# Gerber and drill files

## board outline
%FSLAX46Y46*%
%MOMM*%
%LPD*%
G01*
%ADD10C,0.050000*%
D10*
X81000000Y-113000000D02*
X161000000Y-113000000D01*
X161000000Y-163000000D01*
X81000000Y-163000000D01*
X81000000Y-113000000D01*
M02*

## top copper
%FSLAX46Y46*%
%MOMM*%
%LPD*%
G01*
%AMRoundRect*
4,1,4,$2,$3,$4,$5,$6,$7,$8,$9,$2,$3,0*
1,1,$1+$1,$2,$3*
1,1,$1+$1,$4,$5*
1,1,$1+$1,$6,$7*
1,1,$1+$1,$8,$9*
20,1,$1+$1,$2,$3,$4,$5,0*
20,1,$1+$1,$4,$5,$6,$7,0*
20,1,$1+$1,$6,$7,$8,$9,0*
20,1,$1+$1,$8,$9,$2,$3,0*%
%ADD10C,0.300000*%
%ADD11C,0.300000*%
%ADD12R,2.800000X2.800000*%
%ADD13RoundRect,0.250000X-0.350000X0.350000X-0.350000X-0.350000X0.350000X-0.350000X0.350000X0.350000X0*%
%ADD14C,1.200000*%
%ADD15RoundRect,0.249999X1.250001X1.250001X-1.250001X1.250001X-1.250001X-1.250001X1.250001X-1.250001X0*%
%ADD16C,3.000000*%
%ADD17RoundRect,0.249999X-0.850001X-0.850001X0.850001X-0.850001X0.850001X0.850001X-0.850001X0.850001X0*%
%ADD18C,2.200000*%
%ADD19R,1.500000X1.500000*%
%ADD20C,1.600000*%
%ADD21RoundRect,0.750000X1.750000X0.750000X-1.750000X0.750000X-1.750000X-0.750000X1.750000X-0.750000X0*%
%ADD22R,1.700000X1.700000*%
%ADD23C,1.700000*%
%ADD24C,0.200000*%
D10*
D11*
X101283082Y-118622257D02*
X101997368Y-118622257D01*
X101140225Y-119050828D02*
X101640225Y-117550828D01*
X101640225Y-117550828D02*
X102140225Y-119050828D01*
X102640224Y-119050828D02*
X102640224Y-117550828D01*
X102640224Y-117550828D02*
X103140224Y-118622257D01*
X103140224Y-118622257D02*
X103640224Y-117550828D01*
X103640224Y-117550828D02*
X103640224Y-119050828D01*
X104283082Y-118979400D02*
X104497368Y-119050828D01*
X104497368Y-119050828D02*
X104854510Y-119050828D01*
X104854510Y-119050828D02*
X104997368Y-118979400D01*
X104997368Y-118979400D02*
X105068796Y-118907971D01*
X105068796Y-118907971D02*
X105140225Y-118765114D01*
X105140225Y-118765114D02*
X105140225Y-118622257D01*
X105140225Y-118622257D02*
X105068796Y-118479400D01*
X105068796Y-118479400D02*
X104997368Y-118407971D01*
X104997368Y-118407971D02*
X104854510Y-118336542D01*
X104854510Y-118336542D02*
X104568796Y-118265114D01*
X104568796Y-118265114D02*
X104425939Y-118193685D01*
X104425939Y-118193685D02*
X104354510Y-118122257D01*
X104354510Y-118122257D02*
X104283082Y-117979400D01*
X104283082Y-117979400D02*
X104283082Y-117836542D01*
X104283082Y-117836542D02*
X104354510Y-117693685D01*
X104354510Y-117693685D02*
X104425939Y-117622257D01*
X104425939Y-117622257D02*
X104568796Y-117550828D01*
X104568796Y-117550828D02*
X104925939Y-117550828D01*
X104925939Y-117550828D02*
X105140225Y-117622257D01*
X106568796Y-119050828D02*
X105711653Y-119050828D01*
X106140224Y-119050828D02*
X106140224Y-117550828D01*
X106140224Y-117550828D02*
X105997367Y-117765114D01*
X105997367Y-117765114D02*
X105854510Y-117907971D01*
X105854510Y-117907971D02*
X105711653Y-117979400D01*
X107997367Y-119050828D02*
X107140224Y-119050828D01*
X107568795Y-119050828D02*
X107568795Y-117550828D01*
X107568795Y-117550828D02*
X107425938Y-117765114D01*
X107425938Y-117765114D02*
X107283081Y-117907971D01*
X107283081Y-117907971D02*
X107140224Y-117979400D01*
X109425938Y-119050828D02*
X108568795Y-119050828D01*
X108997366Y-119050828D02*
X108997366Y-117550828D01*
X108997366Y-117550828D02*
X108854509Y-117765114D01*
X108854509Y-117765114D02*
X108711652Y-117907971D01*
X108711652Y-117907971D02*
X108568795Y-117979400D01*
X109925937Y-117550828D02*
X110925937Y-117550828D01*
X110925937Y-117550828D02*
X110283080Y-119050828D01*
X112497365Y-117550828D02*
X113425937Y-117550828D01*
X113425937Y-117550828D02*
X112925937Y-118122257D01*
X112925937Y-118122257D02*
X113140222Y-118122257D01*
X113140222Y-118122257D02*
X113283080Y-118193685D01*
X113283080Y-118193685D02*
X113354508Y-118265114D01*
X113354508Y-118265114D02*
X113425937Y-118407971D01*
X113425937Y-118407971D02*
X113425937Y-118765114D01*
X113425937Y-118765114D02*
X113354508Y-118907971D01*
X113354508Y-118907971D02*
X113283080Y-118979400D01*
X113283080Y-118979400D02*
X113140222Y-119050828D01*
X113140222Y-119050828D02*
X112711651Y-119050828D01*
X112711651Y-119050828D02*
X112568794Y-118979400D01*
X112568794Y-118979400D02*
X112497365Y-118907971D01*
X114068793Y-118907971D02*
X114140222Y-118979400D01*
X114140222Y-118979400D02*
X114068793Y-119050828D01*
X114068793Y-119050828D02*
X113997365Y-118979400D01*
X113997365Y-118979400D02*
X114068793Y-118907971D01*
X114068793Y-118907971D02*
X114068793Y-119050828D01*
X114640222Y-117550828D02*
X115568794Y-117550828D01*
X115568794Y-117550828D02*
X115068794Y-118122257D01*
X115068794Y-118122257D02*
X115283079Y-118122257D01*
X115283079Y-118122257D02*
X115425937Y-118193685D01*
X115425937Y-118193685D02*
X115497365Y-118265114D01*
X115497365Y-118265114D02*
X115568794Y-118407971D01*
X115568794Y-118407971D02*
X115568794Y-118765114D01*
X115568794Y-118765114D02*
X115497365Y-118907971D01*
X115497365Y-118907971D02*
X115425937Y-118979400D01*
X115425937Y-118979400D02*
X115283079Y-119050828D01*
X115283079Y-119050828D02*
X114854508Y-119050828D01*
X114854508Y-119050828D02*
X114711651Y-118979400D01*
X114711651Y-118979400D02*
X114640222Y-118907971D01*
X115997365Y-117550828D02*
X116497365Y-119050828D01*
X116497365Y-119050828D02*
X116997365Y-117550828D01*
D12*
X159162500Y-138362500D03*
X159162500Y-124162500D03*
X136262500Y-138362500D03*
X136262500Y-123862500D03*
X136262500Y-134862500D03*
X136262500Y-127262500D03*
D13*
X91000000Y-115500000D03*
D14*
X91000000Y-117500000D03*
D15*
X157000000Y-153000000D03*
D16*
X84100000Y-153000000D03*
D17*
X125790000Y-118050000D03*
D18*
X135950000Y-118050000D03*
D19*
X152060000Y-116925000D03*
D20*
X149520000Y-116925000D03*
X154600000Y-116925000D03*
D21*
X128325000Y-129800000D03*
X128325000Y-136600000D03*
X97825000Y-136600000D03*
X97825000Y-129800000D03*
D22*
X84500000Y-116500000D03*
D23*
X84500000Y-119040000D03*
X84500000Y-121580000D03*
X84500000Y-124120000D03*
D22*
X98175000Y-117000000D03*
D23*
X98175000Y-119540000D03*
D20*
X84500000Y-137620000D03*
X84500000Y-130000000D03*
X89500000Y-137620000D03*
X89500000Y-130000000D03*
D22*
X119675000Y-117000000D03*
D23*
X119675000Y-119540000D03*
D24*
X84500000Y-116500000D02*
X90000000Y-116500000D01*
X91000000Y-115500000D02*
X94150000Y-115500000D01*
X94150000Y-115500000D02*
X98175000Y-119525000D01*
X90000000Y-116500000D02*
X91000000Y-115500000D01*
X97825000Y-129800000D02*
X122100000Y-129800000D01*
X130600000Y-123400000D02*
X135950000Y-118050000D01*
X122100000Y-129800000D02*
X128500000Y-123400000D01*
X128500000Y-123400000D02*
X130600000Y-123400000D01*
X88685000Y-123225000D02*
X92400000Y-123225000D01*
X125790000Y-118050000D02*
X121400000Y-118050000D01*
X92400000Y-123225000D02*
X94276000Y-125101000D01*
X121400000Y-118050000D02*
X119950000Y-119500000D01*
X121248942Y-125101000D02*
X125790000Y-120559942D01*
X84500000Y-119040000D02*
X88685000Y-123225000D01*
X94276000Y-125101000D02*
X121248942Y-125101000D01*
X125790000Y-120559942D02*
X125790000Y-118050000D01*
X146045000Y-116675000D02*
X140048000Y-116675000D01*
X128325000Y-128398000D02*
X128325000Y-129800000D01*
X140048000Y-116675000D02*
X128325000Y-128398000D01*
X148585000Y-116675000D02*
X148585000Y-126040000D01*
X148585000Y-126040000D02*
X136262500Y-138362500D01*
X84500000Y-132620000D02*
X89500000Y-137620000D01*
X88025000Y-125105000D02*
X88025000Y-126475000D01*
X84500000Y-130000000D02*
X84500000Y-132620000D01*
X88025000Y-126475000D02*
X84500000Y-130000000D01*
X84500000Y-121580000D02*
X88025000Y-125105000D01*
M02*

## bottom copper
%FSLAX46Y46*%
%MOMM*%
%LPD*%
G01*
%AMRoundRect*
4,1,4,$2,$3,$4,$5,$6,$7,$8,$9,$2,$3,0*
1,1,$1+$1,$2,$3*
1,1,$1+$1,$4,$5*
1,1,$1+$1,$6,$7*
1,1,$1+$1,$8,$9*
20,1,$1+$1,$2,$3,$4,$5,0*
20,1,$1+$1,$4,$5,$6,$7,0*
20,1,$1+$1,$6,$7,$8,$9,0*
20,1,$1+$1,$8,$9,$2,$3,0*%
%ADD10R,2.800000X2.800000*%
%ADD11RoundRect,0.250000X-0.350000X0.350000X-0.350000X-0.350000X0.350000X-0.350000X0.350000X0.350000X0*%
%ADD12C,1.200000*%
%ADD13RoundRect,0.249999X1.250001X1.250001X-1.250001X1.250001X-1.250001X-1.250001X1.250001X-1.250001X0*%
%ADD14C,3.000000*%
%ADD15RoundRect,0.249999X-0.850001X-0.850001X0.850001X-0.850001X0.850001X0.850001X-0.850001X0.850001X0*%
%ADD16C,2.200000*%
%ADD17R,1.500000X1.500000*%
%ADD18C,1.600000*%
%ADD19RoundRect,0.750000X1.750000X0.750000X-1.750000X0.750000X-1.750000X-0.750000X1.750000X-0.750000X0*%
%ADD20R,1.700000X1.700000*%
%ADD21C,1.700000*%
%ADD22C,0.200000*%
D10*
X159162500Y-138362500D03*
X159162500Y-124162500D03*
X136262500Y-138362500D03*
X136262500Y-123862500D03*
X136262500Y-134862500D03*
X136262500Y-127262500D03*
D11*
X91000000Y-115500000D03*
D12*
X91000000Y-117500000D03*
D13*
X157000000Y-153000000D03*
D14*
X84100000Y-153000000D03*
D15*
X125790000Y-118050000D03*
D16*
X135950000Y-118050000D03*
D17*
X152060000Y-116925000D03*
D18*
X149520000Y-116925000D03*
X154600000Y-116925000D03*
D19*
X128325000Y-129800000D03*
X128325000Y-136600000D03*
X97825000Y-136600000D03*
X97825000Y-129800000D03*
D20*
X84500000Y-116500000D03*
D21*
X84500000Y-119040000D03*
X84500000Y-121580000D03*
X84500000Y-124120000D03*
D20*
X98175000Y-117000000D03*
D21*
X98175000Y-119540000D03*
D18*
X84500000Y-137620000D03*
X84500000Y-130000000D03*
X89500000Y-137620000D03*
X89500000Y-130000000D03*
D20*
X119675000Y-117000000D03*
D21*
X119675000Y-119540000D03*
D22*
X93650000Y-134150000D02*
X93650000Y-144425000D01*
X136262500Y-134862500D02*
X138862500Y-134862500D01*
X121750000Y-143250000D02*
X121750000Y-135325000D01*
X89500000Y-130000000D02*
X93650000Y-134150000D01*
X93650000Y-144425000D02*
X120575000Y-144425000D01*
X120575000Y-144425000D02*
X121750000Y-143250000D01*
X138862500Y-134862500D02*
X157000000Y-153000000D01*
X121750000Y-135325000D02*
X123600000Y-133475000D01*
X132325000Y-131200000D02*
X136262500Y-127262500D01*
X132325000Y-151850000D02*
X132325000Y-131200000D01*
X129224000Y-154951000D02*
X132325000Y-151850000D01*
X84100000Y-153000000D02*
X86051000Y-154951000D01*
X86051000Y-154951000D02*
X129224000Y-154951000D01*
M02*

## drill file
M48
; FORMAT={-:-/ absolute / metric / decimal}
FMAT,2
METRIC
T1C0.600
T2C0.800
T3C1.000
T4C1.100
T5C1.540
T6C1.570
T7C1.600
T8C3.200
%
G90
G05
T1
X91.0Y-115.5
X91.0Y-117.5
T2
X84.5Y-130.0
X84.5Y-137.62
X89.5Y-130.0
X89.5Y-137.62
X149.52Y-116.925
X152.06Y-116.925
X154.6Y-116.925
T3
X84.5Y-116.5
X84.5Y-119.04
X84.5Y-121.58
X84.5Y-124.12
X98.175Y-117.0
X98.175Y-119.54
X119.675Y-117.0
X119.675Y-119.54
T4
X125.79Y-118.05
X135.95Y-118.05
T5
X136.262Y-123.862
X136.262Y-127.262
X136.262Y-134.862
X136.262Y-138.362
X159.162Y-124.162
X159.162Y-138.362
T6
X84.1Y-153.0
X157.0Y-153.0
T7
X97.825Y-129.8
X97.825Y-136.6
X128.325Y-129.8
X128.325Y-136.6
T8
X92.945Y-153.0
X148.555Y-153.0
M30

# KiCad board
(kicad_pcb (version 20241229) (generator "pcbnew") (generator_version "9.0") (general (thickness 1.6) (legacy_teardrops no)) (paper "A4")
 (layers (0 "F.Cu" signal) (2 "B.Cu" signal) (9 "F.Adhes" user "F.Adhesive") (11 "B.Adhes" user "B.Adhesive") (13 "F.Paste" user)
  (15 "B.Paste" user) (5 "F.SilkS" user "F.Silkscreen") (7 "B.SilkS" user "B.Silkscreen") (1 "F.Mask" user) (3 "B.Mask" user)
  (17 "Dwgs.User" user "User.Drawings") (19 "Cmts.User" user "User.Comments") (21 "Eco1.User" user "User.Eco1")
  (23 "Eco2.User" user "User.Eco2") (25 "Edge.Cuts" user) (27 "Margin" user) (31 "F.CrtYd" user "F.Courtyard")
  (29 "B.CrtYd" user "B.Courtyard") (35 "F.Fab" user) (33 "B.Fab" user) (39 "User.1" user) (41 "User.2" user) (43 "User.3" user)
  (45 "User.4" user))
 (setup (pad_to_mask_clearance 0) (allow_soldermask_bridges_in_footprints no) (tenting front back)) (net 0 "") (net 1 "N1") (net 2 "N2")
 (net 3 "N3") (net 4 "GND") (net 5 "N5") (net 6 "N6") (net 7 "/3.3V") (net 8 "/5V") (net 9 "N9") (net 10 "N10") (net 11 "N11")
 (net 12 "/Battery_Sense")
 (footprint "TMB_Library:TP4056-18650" (layer "F.Cu") (at 160.8625 140.0625 180)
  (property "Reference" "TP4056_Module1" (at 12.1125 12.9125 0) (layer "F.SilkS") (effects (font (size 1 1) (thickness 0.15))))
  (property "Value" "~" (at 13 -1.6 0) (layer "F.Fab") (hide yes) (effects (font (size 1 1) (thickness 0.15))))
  (pad "1" thru_hole rect (at 1.7 1.7 180) (size 2.8 2.8) (drill 1.54) (layers "*.Cu" "*.Mask") (remove_unused_layers no) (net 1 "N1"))
  (pad "2" thru_hole rect (at 1.7 15.9 180) (size 2.8 2.8) (drill 1.54) (layers "*.Cu" "*.Mask") (remove_unused_layers no) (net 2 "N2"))
  (pad "3" thru_hole rect (at 24.6 1.7 180) (size 2.8 2.8) (drill 1.54) (layers "*.Cu" "*.Mask") (remove_unused_layers no) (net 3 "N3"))
  (pad "4" thru_hole rect (at 24.6 16.2 180) (size 2.8 2.8) (drill 1.54) (layers "*.Cu" "*.Mask") (remove_unused_layers no) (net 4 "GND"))
  (pad "5" thru_hole rect (at 24.6 5.2 180) (size 2.8 2.8) (drill 1.54) (layers "*.Cu" "*.Mask") (remove_unused_layers no) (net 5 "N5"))
  (pad "6" thru_hole rect (at 24.6 12.8 180) (size 2.8 2.8) (drill 1.54) (layers "*.Cu" "*.Mask") (remove_unused_layers no) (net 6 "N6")))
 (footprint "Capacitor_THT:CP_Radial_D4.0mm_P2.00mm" (layer "F.Cu") (at 91 115.5 -90)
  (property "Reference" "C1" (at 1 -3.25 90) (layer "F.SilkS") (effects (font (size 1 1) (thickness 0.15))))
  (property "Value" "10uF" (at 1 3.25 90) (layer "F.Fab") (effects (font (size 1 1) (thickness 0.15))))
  (pad "1" thru_hole roundrect (at 0 0 270) (size 1.2 1.2) (drill 0.6) (layers "*.Cu" "*.Mask") (remove_unused_layers no)
   (roundrect_rratio 0.208333) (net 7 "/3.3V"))
  (pad "2" thru_hole circle (at 2 0 270) (size 1.2 1.2) (drill 0.6) (layers "*.Cu" "*.Mask") (remove_unused_layers no) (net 4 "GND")))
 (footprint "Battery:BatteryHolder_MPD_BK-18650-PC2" (layer "F.Cu") (at 157 153 180)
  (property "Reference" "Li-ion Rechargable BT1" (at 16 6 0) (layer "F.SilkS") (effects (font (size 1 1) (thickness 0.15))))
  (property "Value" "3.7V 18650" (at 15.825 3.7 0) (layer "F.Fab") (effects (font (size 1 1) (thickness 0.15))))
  (pad "" np_thru_hole circle (at 8.445 0 180) (size 3.2 3.2) (drill 3.2) (layers "*.Cu" "*.Mask"))
  (pad "" np_thru_hole circle (at 64.055 0 180) (size 3.2 3.2) (drill 3.2) (layers "*.Cu" "*.Mask"))
  (pad "1" thru_hole roundrect (at 0 0 180) (size 3 3) (drill 1.57) (layers "*.Cu" "*.Mask") (remove_unused_layers no)
   (roundrect_rratio 0.083333) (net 5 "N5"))
  (pad "2" thru_hole circle (at 72.9 0 180) (size 3 3) (drill 1.57) (layers "*.Cu" "*.Mask") (remove_unused_layers no) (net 6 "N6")))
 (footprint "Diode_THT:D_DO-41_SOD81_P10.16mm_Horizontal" (layer "F.Cu") (at 125.79 118.05)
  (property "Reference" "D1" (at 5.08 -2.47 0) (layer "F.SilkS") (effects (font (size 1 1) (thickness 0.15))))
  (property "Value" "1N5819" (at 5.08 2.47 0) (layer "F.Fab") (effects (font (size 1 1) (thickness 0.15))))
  (pad "1" thru_hole roundrect (at 0 0) (size 2.2 2.2) (drill 1.1) (layers "*.Cu" "*.Mask") (remove_unused_layers no)
   (roundrect_rratio 0.113636) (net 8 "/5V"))
  (pad "2" thru_hole circle (at 10.16 0) (size 2.2 2.2) (drill 1.1) (layers "*.Cu" "*.Mask") (remove_unused_layers no) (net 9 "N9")))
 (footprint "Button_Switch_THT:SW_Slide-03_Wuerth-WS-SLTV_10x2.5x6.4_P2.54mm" (layer "F.Cu") (at 152.06 116.925)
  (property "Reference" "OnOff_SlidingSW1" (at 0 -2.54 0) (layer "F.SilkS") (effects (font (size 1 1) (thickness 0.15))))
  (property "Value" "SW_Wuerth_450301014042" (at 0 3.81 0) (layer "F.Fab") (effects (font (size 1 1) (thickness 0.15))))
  (pad "1" thru_hole rect (at 0 0) (size 1.5 1.5) (drill 0.8) (layers "*.Cu" "*.Mask") (remove_unused_layers no) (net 3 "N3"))
  (pad "2" thru_hole circle (at -2.54 0) (size 1.6 1.6) (drill 0.8) (layers "*.Cu" "*.Mask") (remove_unused_layers no) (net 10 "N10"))
  (pad "3" thru_hole circle (at 2.54 0) (size 1.6 1.6) (drill 0.8) (layers "*.Cu" "*.Mask") (remove_unused_layers no) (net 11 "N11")))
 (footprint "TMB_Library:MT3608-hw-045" (layer "F.Cu") (at 113.325 132.7 180)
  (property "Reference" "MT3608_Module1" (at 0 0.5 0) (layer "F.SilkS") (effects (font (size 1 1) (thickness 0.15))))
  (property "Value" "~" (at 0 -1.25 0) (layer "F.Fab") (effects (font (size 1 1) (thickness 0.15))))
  (pad "1" thru_hole roundrect (at -15 2.9 180) (size 5 3) (drill 1.6) (layers "*.Cu" "*.Mask") (remove_unused_layers no)
   (roundrect_rratio 0.25) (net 10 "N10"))
  (pad "2" thru_hole roundrect (at -15 -3.9 180) (size 5 3) (drill 1.6) (layers "*.Cu" "*.Mask") (remove_unused_layers no)
   (roundrect_rratio 0.25) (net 4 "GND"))
  (pad "3" thru_hole roundrect (at 15.5 -3.9 180) (size 5 3) (drill 1.6) (layers "*.Cu" "*.Mask") (remove_unused_layers no)
   (roundrect_rratio 0.25) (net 4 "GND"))
  (pad "4" thru_hole roundrect (at 15.5 2.9 180) (size 5 3) (drill 1.6) (layers "*.Cu" "*.Mask") (remove_unused_layers no)
   (roundrect_rratio 0.25) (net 9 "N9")))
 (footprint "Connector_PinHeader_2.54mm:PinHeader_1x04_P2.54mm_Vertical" (layer "F.Cu") (at 84.5 116.5)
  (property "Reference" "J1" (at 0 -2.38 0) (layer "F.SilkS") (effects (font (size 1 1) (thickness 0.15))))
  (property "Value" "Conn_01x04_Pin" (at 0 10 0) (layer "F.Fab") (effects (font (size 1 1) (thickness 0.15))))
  (pad "1" thru_hole rect (at 0 0) (size 1.7 1.7) (drill 1) (layers "*.Cu" "*.Mask") (remove_unused_layers no) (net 7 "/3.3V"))
  (pad "2" thru_hole circle (at 0 2.54) (size 1.7 1.7) (drill 1) (layers "*.Cu" "*.Mask") (remove_unused_layers no) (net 8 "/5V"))
  (pad "3" thru_hole circle (at 0 5.08) (size 1.7 1.7) (drill 1) (layers "*.Cu" "*.Mask") (remove_unused_layers no)
   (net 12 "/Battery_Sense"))
  (pad "4" thru_hole circle (at 0 7.62) (size 1.7 1.7) (drill 1) (layers "*.Cu" "*.Mask") (remove_unused_layers no) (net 4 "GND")))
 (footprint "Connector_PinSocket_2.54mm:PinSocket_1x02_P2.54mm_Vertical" (layer "F.Cu") (at 98.175 117)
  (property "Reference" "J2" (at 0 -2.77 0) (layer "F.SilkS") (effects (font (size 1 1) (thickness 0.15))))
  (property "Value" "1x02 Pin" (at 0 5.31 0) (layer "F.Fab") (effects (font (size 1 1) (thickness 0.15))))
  (pad "1" thru_hole rect (at 0 0) (size 1.7 1.7) (drill 1) (layers "*.Cu" "*.Mask") (remove_unused_layers no) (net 4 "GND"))
  (pad "2" thru_hole circle (at 0 2.54) (size 1.7 1.7) (drill 1) (layers "*.Cu" "*.Mask") (remove_unused_layers no) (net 7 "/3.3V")))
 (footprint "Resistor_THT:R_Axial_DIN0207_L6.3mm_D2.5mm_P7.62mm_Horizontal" (layer "F.Cu") (at 84.5 137.62 90)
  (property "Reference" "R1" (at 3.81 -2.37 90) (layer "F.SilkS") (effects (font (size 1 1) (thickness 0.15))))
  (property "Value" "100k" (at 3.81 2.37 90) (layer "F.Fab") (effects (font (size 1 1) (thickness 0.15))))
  (pad "1" thru_hole circle (at 0 0 90) (size 1.6 1.6) (drill 0.8) (layers "*.Cu" "*.Mask") (remove_unused_layers no) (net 4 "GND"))
  (pad "2" thru_hole circle (at 7.62 0 90) (size 1.6 1.6) (drill 0.8) (layers "*.Cu" "*.Mask") (remove_unused_layers no)
   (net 12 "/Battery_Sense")))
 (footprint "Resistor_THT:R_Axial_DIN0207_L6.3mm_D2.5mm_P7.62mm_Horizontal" (layer "F.Cu") (at 89.5 137.62 90)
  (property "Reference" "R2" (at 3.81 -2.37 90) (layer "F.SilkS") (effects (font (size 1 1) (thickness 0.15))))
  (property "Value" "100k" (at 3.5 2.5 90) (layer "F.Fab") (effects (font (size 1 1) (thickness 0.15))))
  (pad "1" thru_hole circle (at 0 0 90) (size 1.6 1.6) (drill 0.8) (layers "*.Cu" "*.Mask") (remove_unused_layers no)
   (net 12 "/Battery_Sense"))
  (pad "2" thru_hole circle (at 7.62 0 90) (size 1.6 1.6) (drill 0.8) (layers "*.Cu" "*.Mask") (remove_unused_layers no) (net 5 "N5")))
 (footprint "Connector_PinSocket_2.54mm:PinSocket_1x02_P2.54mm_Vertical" (layer "F.Cu") (at 119.675 117)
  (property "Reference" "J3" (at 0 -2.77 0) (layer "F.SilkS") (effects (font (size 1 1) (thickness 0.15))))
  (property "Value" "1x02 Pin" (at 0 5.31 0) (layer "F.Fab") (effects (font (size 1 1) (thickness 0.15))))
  (pad "1" thru_hole rect (at 0 0) (size 1.7 1.7) (drill 1) (layers "*.Cu" "*.Mask") (remove_unused_layers no) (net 4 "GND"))
  (pad "2" thru_hole circle (at 0 2.54) (size 1.7 1.7) (drill 1) (layers "*.Cu" "*.Mask") (remove_unused_layers no) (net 8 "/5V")))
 (gr_rect (start 81 113) (end 161 163) (stroke (width 0.05) (type solid)) (fill no) (layer "Edge.Cuts"))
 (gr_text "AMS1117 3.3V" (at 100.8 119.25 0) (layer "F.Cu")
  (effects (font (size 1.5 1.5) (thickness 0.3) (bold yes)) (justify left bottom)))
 (segment (start 84.5 116.5) (end 90 116.5) (width 0.2) (layer "F.Cu") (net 7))
 (segment (start 91 115.5) (end 94.15 115.5) (width 0.2) (layer "F.Cu") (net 7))
 (segment (start 94.15 115.5) (end 98.175 119.525) (width 0.2) (layer "F.Cu") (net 7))
 (segment (start 90 116.5) (end 91 115.5) (width 0.2) (layer "F.Cu") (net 7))
 (segment (start 97.825 129.8) (end 122.1 129.8) (width 0.2) (layer "F.Cu") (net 9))
 (segment (start 130.6 123.4) (end 135.95 118.05) (width 0.2) (layer "F.Cu") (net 9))
 (segment (start 122.1 129.8) (end 128.5 123.4) (width 0.2) (layer "F.Cu") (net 9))
 (segment (start 128.5 123.4) (end 130.6 123.4) (width 0.2) (layer "F.Cu") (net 9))
 (segment (start 88.685 123.225) (end 92.4 123.225) (width 0.2) (layer "F.Cu") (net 8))
 (segment (start 125.79 118.05) (end 121.4 118.05) (width 0.2) (layer "F.Cu") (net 8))
 (segment (start 92.4 123.225) (end 94.276 125.101) (width 0.2) (layer "F.Cu") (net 8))
 (segment (start 121.4 118.05) (end 119.95 119.5) (width 0.2) (layer "F.Cu") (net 8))
 (segment (start 121.248942 125.101) (end 125.79 120.559942) (width 0.2) (layer "F.Cu") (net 8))
 (segment (start 84.5 119.04) (end 88.685 123.225) (width 0.2) (layer "F.Cu") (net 8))
 (segment (start 94.276 125.101) (end 121.248942 125.101) (width 0.2) (layer "F.Cu") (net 8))
 (segment (start 125.79 120.559942) (end 125.79 118.05) (width 0.2) (layer "F.Cu") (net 8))
 (segment (start 93.65 134.15) (end 93.65 144.425) (width 0.2) (layer "B.Cu") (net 5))
 (segment (start 136.2625 134.8625) (end 138.8625 134.8625) (width 0.2) (layer "B.Cu") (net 5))
 (segment (start 121.75 143.25) (end 121.75 135.325) (width 0.2) (layer "B.Cu") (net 5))
 (segment (start 89.5 130) (end 93.65 134.15) (width 0.2) (layer "B.Cu") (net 5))
 (segment (start 93.65 144.425) (end 120.575 144.425) (width 0.2) (layer "B.Cu") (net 5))
 (segment (start 120.575 144.425) (end 121.75 143.25) (width 0.2) (layer "B.Cu") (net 5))
 (segment (start 138.8625 134.8625) (end 157 153) (width 0.2) (layer "B.Cu") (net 5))
 (segment (start 121.75 135.325) (end 123.6 133.475) (width 0.2) (layer "B.Cu") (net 5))
 (segment (start 132.325 131.2) (end 136.2625 127.2625) (width 0.2) (layer "B.Cu") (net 6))
 (segment (start 132.325 151.85) (end 132.325 131.2) (width 0.2) (layer "B.Cu") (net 6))
 (segment (start 129.224 154.951) (end 132.325 151.85) (width 0.2) (layer "B.Cu") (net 6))
 (segment (start 84.1 153) (end 86.051 154.951) (width 0.2) (layer "B.Cu") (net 6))
 (segment (start 86.051 154.951) (end 129.224 154.951) (width 0.2) (layer "B.Cu") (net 6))
 (segment (start 146.045 116.675) (end 140.048 116.675) (width 0.2) (layer "F.Cu") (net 10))
 (segment (start 128.325 128.398) (end 128.325 129.8) (width 0.2) (layer "F.Cu") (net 10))
 (segment (start 140.048 116.675) (end 128.325 128.398) (width 0.2) (layer "F.Cu") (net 10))
 (segment (start 148.585 116.675) (end 148.585 126.04) (width 0.2) (layer "F.Cu") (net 3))
 (segment (start 148.585 126.04) (end 136.2625 138.3625) (width 0.2) (layer "F.Cu") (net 3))
 (segment (start 84.5 132.62) (end 89.5 137.62) (width 0.2) (layer "F.Cu") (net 12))
 (segment (start 88.025 125.105) (end 88.025 126.475) (width 0.2) (layer "F.Cu") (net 12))
 (segment (start 84.5 130) (end 84.5 132.62) (width 0.2) (layer "F.Cu") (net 12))
 (segment (start 88.025 126.475) (end 84.5 130) (width 0.2) (layer "F.Cu") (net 12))
 (segment (start 84.5 121.58) (end 88.025 125.105) (width 0.2) (layer "F.Cu") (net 12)))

